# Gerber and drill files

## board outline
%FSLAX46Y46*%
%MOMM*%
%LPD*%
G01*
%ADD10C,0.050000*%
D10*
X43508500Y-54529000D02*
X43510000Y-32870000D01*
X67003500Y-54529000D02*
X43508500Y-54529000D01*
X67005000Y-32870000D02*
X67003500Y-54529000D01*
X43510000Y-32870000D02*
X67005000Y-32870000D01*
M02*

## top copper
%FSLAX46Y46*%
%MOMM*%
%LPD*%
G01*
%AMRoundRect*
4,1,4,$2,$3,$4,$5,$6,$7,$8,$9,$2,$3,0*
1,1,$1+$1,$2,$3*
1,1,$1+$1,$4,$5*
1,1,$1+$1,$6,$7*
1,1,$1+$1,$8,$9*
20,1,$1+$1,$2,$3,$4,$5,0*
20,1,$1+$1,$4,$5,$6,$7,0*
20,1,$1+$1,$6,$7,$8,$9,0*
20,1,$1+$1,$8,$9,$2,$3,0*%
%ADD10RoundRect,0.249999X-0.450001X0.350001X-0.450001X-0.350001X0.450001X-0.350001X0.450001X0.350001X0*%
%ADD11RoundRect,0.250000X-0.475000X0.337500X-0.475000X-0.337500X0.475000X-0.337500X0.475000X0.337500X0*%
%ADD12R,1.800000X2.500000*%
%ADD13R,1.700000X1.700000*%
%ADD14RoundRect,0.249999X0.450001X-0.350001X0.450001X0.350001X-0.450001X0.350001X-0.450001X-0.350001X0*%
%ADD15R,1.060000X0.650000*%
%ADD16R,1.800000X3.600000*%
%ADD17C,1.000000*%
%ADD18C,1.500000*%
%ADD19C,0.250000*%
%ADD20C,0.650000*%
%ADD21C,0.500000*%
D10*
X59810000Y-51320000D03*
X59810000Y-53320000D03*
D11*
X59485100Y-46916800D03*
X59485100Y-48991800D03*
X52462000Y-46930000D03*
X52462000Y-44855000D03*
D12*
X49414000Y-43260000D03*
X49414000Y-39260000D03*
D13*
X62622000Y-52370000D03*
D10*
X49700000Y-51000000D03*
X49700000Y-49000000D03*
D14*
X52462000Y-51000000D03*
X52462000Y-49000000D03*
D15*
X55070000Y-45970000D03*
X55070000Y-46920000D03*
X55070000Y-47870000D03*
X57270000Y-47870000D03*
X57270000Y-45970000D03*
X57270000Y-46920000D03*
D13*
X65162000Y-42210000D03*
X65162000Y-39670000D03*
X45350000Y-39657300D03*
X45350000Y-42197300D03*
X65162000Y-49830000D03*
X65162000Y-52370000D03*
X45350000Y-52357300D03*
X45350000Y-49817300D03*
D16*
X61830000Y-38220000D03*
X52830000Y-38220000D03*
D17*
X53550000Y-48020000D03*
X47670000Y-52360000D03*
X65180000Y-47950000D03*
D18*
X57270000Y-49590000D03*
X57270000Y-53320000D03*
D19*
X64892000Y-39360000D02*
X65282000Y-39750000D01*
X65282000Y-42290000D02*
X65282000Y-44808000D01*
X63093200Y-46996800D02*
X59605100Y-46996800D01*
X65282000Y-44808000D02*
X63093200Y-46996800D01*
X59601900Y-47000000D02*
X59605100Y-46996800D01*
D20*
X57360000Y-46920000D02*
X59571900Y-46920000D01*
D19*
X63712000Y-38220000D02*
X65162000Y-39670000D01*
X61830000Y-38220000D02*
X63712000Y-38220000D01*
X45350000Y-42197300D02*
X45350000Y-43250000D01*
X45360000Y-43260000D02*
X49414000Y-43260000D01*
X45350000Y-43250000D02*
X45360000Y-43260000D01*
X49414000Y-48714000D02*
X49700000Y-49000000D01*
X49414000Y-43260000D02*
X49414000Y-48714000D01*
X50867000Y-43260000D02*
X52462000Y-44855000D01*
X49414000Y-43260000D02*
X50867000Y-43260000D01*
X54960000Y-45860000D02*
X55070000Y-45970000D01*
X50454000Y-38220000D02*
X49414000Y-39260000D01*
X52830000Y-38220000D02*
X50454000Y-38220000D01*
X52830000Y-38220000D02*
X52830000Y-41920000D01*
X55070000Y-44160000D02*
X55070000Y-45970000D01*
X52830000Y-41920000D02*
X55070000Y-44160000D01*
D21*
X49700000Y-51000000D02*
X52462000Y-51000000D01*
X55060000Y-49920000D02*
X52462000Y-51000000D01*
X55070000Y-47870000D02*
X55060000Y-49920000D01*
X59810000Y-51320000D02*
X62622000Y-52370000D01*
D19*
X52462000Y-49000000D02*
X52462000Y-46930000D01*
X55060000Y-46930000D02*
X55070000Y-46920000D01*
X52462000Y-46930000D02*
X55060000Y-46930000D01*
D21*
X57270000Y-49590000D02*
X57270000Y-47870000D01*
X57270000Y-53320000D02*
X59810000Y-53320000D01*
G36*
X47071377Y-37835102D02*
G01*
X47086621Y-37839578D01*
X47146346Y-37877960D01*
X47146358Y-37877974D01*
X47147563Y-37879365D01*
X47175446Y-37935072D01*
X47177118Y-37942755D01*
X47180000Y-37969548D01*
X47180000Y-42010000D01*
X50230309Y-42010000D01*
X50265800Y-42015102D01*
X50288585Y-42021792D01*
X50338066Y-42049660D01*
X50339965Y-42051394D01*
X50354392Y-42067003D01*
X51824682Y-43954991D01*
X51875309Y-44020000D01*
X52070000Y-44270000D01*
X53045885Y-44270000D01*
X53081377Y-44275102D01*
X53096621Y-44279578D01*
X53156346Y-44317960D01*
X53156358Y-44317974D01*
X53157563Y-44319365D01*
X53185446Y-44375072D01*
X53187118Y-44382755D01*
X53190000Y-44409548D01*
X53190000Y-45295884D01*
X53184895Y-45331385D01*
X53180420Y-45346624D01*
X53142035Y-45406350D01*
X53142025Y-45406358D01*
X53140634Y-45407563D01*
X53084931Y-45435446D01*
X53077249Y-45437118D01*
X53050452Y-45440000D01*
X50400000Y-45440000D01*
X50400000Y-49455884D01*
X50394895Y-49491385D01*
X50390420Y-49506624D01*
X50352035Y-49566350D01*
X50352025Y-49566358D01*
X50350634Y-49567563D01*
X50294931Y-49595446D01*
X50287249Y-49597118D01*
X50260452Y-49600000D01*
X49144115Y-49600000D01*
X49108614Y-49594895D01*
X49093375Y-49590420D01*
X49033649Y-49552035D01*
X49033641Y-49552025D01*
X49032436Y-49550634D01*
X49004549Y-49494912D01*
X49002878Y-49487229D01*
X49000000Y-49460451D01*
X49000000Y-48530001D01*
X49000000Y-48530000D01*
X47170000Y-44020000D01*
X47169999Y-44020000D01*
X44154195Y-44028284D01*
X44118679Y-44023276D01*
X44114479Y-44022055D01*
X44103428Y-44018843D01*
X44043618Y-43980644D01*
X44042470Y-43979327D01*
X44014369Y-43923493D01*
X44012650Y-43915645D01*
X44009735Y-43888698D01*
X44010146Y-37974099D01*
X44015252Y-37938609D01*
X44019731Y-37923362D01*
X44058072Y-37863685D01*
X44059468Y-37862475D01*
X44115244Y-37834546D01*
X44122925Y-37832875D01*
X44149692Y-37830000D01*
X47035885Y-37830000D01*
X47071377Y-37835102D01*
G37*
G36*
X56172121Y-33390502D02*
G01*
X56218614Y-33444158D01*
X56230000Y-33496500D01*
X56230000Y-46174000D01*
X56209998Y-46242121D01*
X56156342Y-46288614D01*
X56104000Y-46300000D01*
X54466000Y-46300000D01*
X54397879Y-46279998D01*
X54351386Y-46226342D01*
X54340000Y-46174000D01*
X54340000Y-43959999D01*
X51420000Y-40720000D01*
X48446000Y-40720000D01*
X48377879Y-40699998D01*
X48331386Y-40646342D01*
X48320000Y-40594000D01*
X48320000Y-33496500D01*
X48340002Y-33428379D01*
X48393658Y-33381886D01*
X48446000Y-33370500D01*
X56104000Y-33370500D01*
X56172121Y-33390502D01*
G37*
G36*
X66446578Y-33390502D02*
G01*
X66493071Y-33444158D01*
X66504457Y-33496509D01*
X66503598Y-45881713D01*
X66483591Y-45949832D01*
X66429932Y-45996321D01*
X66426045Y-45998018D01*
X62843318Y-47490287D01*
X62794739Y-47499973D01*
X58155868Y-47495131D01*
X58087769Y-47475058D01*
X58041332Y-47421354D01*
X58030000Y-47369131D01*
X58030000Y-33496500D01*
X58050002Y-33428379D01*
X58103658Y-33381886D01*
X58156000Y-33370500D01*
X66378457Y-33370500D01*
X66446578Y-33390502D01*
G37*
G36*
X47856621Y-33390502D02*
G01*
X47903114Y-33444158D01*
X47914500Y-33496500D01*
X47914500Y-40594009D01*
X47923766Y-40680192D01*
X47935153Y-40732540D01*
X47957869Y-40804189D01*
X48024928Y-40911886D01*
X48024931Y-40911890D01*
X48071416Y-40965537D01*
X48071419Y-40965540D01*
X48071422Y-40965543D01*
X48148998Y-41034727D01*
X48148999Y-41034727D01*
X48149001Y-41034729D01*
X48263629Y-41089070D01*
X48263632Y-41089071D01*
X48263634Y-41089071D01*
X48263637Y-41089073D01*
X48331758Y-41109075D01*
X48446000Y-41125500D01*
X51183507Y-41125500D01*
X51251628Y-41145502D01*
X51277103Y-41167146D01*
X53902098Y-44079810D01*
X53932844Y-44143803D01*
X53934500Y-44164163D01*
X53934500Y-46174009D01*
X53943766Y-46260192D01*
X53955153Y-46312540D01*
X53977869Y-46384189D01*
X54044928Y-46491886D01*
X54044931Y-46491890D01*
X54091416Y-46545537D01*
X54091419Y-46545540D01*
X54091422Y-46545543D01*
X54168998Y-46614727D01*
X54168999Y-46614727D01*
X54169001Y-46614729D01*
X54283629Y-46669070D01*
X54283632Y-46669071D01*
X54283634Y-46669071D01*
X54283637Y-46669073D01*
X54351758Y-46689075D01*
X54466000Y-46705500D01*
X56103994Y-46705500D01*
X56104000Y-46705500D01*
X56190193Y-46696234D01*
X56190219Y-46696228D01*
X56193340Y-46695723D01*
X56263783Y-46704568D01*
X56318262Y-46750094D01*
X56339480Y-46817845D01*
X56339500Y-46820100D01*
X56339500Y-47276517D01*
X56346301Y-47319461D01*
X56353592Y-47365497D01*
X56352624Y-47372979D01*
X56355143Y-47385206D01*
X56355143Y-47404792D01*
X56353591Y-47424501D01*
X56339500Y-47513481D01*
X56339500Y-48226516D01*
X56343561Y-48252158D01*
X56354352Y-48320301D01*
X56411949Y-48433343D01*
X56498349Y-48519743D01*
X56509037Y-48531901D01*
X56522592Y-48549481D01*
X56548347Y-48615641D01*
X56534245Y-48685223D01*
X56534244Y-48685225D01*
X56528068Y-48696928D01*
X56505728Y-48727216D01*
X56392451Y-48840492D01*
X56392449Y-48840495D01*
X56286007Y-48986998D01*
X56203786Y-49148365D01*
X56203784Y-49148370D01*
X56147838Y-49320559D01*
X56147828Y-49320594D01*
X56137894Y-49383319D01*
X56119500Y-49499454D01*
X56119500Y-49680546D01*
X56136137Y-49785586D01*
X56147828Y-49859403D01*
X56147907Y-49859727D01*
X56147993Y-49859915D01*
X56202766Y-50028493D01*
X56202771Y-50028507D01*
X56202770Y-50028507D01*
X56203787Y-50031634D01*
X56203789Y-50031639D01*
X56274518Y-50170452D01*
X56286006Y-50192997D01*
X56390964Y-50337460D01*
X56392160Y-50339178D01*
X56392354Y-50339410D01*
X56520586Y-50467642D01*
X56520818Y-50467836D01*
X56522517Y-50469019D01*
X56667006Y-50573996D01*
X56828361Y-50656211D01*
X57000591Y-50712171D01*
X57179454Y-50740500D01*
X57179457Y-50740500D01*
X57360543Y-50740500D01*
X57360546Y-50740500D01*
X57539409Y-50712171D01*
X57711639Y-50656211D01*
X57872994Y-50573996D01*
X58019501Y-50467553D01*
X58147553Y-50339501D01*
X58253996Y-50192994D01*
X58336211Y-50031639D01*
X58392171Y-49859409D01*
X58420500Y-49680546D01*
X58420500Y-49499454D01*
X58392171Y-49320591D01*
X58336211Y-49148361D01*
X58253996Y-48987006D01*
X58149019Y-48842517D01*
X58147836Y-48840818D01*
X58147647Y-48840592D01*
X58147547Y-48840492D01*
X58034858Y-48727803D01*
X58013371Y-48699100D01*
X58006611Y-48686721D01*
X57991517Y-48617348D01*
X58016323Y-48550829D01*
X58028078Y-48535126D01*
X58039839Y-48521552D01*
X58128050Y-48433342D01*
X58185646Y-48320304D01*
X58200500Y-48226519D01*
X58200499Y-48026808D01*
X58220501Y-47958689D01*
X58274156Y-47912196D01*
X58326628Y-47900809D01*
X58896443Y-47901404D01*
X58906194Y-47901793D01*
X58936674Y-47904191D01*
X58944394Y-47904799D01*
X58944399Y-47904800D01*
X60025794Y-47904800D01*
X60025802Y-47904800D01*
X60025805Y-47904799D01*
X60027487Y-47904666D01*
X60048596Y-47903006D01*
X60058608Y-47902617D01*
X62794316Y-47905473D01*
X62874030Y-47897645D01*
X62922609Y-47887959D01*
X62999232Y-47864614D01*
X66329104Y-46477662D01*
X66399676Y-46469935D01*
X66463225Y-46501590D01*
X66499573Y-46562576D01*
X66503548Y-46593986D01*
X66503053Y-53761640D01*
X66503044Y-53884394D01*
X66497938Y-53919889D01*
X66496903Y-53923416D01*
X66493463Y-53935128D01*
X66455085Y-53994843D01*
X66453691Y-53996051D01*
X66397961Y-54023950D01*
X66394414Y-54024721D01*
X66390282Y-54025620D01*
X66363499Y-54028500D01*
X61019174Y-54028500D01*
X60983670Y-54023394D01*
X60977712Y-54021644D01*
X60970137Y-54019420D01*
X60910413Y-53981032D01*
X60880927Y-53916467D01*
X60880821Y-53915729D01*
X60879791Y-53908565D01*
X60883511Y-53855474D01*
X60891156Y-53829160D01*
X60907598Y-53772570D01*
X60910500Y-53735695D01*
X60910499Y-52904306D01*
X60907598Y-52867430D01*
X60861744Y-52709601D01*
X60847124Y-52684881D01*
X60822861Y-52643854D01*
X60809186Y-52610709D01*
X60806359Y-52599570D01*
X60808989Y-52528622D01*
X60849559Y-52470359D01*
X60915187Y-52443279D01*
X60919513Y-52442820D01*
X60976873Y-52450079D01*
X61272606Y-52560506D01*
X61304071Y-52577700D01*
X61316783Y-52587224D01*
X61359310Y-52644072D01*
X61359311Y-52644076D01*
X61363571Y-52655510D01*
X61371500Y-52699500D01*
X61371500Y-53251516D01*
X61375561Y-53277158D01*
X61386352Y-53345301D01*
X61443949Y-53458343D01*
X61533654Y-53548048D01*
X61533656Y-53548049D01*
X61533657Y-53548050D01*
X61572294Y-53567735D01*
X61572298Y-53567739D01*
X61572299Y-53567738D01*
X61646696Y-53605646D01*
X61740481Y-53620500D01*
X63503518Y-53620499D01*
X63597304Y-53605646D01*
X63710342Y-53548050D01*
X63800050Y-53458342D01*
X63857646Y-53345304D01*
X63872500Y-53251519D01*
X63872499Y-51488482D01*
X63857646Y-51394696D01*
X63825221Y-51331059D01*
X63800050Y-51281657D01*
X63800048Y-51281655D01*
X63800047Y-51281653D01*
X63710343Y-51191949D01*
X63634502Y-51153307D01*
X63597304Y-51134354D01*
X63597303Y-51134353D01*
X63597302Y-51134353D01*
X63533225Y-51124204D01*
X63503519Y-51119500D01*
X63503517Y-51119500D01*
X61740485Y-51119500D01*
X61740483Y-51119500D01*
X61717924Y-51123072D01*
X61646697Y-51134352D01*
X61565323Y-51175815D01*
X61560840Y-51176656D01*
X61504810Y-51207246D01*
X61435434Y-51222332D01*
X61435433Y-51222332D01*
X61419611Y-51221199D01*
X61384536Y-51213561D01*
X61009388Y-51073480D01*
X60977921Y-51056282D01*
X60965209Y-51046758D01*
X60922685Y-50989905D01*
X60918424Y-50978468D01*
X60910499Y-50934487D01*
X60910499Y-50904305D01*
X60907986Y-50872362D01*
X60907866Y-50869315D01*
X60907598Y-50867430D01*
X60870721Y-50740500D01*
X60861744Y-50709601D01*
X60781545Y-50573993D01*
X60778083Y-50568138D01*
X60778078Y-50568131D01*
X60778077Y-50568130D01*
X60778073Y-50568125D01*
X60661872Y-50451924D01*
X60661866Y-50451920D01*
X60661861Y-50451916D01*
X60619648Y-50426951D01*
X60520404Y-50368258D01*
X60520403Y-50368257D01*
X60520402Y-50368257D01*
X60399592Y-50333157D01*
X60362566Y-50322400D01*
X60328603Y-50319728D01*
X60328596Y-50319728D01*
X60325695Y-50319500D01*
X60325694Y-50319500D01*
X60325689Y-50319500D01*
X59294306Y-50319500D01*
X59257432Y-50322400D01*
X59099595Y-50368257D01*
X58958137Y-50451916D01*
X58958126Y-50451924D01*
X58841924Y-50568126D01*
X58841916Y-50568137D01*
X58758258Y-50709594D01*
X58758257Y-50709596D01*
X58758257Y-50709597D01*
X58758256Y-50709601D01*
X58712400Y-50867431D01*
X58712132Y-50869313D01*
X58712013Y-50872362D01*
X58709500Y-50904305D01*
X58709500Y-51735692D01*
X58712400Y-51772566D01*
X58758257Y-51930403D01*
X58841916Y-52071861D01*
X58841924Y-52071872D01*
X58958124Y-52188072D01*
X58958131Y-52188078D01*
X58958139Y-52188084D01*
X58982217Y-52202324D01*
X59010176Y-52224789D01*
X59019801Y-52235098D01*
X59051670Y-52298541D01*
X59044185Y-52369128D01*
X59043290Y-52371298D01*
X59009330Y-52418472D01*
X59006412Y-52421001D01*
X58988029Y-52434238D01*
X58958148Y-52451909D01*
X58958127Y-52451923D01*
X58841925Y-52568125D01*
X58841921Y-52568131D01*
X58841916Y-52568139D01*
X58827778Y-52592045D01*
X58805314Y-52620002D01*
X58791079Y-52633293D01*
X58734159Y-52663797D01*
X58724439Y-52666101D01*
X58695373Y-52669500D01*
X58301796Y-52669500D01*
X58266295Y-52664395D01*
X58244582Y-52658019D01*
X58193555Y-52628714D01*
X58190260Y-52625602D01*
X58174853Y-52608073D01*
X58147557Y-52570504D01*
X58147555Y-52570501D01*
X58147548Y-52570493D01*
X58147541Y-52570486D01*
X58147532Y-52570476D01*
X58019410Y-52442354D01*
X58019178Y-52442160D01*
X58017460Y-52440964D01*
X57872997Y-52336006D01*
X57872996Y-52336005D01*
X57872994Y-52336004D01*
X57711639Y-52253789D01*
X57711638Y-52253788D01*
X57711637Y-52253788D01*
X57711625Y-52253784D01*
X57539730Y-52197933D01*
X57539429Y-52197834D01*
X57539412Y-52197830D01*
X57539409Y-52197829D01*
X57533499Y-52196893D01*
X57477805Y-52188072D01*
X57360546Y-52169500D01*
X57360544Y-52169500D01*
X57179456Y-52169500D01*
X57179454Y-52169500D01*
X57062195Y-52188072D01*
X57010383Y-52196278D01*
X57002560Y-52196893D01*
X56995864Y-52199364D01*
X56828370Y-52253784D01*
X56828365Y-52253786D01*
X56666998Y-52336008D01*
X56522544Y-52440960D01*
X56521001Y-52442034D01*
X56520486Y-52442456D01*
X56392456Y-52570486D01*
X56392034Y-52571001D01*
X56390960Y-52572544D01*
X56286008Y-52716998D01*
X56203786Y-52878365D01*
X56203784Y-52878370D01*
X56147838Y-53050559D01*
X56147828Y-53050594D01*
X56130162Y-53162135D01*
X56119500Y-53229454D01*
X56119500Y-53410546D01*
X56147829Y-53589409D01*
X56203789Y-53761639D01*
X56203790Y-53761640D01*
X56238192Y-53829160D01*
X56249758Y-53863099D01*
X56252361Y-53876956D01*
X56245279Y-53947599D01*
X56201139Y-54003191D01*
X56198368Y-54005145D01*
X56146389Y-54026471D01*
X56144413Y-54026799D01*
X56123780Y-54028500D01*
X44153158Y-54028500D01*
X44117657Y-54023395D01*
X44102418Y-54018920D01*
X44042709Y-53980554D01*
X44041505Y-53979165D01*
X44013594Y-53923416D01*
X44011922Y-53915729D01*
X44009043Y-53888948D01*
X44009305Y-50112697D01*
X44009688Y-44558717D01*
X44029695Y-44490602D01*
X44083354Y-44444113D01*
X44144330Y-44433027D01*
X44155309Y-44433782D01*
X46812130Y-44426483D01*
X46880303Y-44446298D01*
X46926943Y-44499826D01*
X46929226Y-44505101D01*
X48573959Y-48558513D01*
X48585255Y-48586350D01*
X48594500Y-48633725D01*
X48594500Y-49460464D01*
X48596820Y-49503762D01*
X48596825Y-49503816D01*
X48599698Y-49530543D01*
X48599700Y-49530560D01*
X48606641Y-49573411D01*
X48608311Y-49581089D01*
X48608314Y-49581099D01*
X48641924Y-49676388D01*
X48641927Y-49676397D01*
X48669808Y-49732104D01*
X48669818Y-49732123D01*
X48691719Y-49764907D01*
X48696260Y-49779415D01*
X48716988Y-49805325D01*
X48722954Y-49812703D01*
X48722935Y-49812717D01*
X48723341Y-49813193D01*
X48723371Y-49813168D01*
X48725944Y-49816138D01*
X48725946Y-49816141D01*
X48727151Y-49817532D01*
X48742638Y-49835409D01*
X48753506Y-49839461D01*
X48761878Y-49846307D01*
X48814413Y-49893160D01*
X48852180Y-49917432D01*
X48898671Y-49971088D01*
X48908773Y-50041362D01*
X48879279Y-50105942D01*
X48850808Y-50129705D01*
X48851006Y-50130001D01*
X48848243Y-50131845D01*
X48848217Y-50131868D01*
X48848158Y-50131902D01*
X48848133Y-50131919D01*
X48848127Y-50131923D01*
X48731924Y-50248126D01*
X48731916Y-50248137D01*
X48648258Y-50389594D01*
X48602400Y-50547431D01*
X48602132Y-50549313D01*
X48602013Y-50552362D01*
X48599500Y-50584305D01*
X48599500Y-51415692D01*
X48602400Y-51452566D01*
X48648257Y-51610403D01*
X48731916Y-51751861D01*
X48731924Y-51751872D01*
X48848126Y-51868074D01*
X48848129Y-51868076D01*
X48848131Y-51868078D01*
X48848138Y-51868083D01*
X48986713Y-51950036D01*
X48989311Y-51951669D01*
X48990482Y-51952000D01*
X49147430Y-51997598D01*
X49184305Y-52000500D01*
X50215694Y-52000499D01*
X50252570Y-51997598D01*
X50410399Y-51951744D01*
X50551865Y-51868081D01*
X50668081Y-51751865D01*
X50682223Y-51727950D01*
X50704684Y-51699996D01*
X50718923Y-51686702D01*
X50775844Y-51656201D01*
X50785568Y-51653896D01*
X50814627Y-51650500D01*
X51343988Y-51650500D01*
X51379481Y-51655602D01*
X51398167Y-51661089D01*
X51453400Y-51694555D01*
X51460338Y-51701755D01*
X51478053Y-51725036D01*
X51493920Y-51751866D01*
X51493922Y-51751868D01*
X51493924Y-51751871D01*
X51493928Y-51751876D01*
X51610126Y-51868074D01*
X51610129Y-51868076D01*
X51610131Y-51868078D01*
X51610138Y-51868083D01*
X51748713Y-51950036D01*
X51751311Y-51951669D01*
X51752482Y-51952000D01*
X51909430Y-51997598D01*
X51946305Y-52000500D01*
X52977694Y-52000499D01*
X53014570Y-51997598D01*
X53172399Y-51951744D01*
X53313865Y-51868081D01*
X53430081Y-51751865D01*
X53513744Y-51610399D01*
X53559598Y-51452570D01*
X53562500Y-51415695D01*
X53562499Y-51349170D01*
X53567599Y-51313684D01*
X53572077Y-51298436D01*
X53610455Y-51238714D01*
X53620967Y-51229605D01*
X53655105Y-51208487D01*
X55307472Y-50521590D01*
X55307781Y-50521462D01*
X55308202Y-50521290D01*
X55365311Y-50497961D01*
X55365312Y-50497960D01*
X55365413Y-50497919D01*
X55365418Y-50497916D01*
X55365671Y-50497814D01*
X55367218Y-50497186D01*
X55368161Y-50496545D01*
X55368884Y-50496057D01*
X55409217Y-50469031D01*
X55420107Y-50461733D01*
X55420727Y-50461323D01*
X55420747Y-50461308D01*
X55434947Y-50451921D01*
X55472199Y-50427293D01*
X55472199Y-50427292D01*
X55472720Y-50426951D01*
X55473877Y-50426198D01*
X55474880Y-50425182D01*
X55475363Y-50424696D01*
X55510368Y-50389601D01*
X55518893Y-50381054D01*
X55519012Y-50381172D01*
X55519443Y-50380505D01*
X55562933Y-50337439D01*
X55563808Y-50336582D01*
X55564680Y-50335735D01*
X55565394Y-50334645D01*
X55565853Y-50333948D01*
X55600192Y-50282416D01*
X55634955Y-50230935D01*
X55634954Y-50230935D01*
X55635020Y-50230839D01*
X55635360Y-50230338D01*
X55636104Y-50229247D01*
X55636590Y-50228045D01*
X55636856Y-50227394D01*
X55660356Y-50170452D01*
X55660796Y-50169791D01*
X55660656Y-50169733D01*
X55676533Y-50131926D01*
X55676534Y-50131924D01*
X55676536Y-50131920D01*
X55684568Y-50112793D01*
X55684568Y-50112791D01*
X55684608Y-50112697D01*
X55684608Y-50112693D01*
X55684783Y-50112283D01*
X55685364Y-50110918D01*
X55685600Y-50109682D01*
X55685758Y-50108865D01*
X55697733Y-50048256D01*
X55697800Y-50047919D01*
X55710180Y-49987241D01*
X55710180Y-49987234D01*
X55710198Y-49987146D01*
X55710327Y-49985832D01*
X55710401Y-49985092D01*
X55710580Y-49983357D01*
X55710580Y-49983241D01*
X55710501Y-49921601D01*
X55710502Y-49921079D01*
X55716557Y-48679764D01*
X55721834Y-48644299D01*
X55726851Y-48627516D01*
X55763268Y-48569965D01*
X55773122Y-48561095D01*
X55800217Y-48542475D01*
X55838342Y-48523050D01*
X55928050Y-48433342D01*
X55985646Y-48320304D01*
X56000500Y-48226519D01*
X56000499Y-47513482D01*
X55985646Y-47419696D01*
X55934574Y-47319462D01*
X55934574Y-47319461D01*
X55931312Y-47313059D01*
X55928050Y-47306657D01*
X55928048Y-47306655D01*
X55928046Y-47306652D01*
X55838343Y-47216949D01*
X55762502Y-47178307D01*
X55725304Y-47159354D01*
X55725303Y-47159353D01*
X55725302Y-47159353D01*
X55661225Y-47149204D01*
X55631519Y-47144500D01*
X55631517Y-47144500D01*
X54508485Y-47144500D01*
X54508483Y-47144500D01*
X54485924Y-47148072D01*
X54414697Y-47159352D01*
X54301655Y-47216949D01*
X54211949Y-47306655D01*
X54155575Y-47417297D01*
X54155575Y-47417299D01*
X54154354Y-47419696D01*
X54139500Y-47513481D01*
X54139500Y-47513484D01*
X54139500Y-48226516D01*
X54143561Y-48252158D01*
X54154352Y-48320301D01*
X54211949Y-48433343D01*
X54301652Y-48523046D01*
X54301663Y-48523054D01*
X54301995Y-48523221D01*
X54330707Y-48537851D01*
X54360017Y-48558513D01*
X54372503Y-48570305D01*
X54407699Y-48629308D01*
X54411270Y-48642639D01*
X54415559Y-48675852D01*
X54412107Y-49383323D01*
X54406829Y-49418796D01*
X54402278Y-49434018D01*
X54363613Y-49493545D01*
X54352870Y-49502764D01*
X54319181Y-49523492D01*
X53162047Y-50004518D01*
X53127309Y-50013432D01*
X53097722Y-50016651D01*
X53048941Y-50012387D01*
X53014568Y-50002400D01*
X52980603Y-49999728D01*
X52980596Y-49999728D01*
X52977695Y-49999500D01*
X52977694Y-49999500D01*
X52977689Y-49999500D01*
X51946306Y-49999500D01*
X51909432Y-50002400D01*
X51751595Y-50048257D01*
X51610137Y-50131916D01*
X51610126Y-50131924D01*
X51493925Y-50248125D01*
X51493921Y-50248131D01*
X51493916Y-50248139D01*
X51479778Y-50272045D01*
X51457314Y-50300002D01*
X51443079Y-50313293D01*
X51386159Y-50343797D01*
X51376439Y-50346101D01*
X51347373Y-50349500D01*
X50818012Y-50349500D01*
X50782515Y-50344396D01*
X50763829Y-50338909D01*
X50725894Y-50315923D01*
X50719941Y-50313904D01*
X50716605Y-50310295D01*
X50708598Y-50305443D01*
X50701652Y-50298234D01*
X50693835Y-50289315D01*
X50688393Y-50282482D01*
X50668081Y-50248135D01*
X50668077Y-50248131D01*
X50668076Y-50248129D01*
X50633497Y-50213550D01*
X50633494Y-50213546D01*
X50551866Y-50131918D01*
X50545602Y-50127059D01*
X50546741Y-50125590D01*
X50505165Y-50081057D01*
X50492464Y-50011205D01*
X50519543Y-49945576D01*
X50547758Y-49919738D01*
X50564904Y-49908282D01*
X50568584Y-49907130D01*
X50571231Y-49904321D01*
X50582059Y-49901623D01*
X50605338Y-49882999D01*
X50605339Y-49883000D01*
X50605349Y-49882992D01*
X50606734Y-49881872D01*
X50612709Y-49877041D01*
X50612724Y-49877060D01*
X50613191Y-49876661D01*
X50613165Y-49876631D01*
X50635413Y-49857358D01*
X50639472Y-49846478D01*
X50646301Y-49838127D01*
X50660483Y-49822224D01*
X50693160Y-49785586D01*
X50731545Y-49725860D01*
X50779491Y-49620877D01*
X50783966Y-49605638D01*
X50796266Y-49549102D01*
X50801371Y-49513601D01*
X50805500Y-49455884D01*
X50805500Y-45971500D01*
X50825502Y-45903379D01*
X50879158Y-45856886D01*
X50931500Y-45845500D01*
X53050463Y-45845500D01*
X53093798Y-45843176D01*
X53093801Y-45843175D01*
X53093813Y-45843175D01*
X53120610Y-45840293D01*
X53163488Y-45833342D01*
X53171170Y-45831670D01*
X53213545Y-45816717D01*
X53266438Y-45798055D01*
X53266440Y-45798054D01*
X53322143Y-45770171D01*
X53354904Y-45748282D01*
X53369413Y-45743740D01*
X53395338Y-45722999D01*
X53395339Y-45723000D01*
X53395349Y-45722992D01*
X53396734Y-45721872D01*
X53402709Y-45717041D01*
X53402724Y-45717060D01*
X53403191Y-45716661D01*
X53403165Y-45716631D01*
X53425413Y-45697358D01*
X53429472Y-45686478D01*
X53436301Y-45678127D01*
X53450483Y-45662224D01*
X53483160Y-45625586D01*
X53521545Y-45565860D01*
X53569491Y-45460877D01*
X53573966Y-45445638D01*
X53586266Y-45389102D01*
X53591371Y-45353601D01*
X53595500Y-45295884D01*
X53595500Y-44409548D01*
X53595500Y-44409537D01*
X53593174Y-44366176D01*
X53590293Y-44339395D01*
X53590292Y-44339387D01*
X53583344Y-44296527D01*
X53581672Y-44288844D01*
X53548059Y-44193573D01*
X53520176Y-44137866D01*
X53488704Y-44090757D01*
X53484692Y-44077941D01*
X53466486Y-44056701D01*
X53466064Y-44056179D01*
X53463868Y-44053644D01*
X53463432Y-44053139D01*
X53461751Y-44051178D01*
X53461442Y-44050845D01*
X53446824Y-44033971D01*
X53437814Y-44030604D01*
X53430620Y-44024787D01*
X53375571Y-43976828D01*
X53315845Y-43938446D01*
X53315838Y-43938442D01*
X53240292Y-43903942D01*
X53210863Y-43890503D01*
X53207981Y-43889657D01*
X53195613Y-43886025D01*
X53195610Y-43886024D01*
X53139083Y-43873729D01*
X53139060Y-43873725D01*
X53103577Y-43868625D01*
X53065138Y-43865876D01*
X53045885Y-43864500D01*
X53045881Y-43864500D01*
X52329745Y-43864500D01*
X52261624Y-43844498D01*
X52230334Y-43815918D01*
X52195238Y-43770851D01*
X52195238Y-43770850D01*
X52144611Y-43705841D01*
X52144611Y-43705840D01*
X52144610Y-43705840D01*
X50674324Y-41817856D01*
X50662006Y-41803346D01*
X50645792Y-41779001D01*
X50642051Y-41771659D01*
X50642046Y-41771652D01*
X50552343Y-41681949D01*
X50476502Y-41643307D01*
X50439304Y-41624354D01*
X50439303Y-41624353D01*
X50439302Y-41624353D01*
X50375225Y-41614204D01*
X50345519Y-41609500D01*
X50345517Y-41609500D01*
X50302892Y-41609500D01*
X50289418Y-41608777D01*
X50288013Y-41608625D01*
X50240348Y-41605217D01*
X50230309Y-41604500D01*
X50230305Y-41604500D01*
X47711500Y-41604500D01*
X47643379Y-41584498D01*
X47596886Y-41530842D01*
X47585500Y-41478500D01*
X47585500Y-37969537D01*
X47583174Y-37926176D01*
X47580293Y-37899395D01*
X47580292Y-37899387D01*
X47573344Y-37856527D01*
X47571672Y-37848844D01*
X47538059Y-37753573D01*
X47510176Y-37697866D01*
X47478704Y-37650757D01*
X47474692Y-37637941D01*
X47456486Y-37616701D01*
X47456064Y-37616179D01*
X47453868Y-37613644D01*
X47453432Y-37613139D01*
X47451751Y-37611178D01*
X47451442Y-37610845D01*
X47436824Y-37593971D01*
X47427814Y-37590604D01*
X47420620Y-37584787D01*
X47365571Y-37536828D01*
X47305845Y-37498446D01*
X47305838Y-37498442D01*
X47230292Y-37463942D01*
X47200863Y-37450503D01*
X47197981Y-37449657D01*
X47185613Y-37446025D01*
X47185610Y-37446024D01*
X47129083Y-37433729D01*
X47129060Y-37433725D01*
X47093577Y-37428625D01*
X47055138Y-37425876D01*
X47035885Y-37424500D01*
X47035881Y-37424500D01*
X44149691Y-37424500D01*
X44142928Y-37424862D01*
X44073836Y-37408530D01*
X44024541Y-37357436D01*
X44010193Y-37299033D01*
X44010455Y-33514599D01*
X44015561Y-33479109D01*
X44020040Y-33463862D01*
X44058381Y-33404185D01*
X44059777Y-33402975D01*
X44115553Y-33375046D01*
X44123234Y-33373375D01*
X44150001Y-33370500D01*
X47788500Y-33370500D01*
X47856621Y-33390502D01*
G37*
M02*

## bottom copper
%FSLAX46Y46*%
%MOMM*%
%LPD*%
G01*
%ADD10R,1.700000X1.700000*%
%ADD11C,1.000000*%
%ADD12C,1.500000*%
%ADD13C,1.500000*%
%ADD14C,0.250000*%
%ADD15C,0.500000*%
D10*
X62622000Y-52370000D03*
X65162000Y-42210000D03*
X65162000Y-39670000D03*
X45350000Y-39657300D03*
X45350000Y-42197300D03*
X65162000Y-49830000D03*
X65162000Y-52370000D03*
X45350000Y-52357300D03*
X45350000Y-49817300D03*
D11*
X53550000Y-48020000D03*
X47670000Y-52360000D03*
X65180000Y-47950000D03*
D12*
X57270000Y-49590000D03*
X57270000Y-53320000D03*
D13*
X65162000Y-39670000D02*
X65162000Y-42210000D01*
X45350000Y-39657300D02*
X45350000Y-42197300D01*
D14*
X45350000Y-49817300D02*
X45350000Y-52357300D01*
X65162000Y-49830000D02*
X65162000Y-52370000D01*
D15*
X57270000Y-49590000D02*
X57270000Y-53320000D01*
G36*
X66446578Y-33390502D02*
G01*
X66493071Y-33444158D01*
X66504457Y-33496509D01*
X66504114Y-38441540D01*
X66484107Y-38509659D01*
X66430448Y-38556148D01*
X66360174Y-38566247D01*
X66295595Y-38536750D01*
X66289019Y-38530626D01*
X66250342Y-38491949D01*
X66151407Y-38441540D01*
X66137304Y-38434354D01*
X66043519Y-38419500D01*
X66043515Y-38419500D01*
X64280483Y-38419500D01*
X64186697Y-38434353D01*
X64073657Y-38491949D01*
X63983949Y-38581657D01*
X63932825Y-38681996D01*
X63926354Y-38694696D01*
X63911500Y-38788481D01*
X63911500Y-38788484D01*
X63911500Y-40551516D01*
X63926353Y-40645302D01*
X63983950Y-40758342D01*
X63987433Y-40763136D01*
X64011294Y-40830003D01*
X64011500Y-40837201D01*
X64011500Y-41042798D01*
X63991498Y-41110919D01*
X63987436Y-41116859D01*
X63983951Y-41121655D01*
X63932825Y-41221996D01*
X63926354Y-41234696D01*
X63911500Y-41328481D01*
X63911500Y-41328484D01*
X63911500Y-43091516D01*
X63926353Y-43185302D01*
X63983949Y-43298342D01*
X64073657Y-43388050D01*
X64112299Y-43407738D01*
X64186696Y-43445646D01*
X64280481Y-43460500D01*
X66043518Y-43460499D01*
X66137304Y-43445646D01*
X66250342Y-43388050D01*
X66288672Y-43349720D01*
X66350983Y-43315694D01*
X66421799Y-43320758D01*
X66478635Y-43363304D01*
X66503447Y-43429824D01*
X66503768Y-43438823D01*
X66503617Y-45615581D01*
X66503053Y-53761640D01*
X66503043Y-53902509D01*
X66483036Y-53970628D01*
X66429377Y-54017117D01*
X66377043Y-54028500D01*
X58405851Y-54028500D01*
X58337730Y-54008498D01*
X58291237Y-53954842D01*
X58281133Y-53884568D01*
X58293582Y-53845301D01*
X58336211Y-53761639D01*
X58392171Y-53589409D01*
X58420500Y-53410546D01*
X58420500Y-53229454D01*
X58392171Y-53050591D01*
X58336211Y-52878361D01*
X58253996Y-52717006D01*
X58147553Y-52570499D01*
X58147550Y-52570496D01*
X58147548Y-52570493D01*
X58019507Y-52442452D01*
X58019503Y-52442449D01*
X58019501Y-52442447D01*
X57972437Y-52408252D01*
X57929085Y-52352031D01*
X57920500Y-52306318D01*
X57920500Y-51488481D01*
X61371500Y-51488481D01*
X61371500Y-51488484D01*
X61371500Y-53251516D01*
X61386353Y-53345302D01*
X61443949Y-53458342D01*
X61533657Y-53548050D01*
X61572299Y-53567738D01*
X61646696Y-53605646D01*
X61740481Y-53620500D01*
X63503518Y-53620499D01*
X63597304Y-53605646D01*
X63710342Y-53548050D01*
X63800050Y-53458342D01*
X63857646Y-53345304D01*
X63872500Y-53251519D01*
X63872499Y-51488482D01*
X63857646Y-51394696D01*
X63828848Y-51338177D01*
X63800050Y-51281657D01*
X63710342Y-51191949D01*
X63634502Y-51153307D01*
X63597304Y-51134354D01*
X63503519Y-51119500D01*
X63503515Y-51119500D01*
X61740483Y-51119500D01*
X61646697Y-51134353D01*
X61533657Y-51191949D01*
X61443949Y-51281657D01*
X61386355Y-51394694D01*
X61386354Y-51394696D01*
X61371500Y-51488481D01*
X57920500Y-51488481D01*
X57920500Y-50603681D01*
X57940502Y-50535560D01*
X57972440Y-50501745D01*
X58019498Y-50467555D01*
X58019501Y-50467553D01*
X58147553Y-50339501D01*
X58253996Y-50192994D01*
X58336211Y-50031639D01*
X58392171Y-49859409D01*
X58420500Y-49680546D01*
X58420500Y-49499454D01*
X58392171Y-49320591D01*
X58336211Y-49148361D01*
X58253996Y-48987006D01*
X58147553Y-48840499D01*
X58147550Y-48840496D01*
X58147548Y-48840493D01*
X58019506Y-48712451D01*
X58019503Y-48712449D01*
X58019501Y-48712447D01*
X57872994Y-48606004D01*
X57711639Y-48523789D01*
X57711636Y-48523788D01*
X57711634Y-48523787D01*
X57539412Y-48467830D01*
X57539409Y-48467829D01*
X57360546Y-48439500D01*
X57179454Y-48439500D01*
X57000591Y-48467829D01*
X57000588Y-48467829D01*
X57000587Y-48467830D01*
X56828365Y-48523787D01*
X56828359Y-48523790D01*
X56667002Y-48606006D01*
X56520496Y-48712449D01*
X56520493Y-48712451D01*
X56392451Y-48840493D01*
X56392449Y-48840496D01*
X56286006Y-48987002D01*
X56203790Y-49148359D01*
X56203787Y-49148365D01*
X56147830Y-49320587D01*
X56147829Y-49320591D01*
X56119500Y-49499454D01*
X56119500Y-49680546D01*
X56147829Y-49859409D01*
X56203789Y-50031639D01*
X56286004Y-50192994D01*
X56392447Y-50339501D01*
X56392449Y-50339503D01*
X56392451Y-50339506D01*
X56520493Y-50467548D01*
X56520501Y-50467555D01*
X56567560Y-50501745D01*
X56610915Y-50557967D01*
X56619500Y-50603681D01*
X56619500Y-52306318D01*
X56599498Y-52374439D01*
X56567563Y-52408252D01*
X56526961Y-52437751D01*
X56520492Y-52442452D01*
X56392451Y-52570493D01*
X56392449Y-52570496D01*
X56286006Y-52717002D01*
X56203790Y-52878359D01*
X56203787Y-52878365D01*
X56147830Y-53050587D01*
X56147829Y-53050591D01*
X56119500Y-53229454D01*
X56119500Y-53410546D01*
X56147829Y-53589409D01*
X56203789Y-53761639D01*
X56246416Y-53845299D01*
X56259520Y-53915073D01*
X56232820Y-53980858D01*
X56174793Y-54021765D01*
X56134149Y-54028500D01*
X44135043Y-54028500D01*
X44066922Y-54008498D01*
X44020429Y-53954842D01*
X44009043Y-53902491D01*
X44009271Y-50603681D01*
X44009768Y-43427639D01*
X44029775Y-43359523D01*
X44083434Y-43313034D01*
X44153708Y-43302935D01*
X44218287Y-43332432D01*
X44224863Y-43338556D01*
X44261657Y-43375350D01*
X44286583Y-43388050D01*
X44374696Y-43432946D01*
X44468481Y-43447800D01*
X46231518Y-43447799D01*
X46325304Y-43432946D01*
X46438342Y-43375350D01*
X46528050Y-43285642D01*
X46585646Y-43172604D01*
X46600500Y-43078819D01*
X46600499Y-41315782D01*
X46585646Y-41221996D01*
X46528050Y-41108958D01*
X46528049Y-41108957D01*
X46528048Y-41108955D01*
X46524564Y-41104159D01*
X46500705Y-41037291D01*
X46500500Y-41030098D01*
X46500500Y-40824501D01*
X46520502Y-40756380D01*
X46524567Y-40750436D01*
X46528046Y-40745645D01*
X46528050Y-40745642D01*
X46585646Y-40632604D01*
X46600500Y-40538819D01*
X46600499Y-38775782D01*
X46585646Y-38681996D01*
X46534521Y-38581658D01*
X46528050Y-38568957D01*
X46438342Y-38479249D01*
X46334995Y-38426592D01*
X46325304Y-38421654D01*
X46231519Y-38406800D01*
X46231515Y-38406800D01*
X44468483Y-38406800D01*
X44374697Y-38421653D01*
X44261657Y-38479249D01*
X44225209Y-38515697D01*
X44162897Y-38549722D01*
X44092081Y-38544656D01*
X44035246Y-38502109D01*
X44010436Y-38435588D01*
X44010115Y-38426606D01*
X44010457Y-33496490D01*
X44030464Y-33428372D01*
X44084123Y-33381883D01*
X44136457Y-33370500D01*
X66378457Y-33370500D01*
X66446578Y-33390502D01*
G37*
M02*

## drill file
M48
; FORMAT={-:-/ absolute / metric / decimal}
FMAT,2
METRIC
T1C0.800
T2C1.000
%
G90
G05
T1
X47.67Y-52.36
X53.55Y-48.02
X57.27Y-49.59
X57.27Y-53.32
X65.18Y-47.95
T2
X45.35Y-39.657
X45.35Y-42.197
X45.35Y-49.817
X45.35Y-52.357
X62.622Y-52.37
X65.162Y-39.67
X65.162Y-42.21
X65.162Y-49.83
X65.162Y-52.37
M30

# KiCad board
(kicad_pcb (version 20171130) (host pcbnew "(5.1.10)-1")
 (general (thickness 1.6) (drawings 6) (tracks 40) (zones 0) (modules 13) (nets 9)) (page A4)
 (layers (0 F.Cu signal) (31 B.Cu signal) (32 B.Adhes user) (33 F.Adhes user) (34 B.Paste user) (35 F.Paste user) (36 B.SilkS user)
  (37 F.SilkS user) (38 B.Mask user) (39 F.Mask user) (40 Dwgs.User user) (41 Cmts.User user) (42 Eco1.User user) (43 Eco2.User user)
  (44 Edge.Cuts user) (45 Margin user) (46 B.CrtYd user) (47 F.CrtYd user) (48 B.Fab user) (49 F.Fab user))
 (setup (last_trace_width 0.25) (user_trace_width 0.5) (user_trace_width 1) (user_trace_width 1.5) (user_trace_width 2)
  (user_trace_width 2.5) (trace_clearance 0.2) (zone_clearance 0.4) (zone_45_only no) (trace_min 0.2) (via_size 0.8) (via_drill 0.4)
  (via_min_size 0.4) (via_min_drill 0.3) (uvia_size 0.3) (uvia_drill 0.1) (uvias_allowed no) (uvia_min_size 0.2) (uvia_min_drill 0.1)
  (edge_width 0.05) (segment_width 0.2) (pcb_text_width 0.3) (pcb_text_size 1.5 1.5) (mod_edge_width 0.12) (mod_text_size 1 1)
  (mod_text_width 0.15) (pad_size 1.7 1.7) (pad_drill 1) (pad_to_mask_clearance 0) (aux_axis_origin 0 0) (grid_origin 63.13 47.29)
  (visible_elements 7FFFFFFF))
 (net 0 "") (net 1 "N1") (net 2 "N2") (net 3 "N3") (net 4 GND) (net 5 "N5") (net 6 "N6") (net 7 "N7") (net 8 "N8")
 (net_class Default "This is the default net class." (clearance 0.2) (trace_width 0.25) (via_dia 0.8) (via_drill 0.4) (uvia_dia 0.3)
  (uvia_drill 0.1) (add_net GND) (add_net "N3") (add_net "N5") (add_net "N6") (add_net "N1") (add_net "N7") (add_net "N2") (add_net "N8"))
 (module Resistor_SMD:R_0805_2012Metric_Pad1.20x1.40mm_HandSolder (layer F.Cu) (at 59.81 52.32 270)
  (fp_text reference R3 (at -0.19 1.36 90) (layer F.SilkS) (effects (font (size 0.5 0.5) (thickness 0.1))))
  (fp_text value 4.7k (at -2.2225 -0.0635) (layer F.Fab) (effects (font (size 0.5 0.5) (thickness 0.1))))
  (pad 1 smd roundrect (at -1 0 270) (size 1.2 1.4) (layers F.Cu F.Paste F.Mask) (roundrect_rratio 0.2083325) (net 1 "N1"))
  (pad 2 smd roundrect (at 1 0 270) (size 1.2 1.4) (layers F.Cu F.Paste F.Mask) (roundrect_rratio 0.2083325) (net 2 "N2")))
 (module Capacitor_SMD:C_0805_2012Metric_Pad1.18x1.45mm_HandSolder (layer F.Cu) (at 59.4851 47.9543 270)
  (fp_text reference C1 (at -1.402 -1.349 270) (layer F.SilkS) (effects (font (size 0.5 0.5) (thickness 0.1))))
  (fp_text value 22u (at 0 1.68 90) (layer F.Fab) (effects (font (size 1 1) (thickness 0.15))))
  (pad 1 smd roundrect (at -1.0375 0 270) (size 1.175 1.45) (layers F.Cu F.Paste F.Mask) (roundrect_rratio 0.2127659574468085) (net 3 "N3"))
  (pad 2 smd roundrect (at 1.0375 0 270) (size 1.175 1.45) (layers F.Cu F.Paste F.Mask) (roundrect_rratio 0.2127659574468085) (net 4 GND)))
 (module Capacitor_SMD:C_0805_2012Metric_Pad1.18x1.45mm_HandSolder (layer F.Cu) (at 52.462 45.8925 270)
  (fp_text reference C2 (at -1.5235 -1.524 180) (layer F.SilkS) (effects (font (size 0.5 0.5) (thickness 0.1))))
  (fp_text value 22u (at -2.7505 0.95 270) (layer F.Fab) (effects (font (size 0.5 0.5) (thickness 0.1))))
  (pad 2 smd roundrect (at 1.0375 0 270) (size 1.175 1.45) (layers F.Cu F.Paste F.Mask) (roundrect_rratio 0.2127659574468085) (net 4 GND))
  (pad 1 smd roundrect (at -1.0375 0 270) (size 1.175 1.45) (layers F.Cu F.Paste F.Mask) (roundrect_rratio 0.2127659574468085) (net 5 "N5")))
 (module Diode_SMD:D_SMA (layer F.Cu) (at 49.414 41.26 90)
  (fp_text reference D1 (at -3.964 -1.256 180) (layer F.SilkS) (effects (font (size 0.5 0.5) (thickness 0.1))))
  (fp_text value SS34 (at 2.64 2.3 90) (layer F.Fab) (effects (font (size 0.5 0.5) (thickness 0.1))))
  (pad 1 smd rect (at -2 0 90) (size 2.5 1.8) (layers F.Cu F.Paste F.Mask) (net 5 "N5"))
  (pad 2 smd rect (at 2 0 90) (size 2.5 1.8) (layers F.Cu F.Paste F.Mask) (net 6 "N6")))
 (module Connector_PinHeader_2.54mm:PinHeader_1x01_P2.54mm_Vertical (layer F.Cu) (at 62.622 52.37 180)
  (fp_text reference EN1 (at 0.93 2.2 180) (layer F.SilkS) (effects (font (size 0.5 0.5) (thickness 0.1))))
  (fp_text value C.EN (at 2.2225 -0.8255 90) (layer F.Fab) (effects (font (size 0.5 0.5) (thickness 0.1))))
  (pad 1 thru_hole rect (at 0 0 180) (size 1.7 1.7) (drill 1) (layers *.Cu *.Mask) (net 1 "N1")))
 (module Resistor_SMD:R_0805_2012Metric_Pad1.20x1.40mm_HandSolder (layer F.Cu) (at 49.7 50 270)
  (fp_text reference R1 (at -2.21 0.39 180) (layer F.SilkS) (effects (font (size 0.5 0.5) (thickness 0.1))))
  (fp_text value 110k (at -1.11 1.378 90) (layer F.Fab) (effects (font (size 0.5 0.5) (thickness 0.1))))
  (pad 2 smd roundrect (at 1 0 270) (size 1.2 1.4) (layers F.Cu F.Paste F.Mask) (roundrect_rratio 0.2083325) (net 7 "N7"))
  (pad 1 smd roundrect (at -1 0 270) (size 1.2 1.4) (layers F.Cu F.Paste F.Mask) (roundrect_rratio 0.2083325) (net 5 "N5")))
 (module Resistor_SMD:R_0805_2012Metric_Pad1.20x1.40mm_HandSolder (layer F.Cu) (at 52.462 50 90)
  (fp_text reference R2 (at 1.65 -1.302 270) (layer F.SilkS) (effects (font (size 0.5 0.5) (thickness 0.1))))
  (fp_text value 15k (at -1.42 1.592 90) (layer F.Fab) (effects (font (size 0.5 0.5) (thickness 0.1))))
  (pad 1 smd roundrect (at -1 0 90) (size 1.2 1.4) (layers F.Cu F.Paste F.Mask) (roundrect_rratio 0.2083325) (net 7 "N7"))
  (pad 2 smd roundrect (at 1 0 90) (size 1.2 1.4) (layers F.Cu F.Paste F.Mask) (roundrect_rratio 0.2083325) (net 4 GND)))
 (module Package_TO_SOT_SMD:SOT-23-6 (layer F.Cu) (at 56.17 46.92) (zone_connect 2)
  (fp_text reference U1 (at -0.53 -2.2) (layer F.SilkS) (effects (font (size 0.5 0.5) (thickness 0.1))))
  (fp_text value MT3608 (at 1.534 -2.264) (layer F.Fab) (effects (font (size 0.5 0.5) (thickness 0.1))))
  (pad 1 smd rect (at -1.1 -0.95) (size 1.06 0.65) (layers F.Cu F.Paste F.Mask) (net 6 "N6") (zone_connect 2))
  (pad 2 smd rect (at -1.1 0) (size 1.06 0.65) (layers F.Cu F.Paste F.Mask) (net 4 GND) (zone_connect 2))
  (pad 3 smd rect (at -1.1 0.95) (size 1.06 0.65) (layers F.Cu F.Paste F.Mask) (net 7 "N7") (zone_connect 2))
  (pad 4 smd rect (at 1.1 0.95) (size 1.06 0.65) (layers F.Cu F.Paste F.Mask) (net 2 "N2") (zone_connect 2))
  (pad 6 smd rect (at 1.1 -0.95) (size 1.06 0.65) (layers F.Cu F.Paste F.Mask) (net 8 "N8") (zone_connect 2))
  (pad 5 smd rect (at 1.1 0) (size 1.06 0.65) (layers F.Cu F.Paste F.Mask) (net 3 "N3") (zone_connect 2)))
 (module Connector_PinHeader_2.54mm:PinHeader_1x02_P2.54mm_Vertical (layer F.Cu) (at 65.162 39.67)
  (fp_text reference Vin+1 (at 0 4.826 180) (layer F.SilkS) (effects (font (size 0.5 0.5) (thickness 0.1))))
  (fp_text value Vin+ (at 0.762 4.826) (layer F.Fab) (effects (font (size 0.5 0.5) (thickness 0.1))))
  (pad 2 thru_hole rect (at 0 2.54) (size 1.7 1.7) (drill 1) (layers *.Cu *.Mask) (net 3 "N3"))
  (pad 1 thru_hole rect (at 0 0) (size 1.7 1.7) (drill 1) (layers *.Cu *.Mask) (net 3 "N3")))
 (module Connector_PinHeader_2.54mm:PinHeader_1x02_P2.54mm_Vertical (layer F.Cu) (at 45.35 39.6573)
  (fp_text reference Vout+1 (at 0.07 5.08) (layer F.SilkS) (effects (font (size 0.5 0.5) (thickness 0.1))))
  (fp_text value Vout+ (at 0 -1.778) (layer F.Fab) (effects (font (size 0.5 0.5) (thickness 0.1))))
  (pad 1 thru_hole rect (at 0 0) (size 1.7 1.7) (drill 1) (layers *.Cu *.Mask) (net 5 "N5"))
  (pad 2 thru_hole rect (at 0 2.54) (size 1.7 1.7) (drill 1) (layers *.Cu *.Mask) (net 5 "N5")))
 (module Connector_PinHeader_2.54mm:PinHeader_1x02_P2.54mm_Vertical (layer F.Cu) (at 65.162 49.83)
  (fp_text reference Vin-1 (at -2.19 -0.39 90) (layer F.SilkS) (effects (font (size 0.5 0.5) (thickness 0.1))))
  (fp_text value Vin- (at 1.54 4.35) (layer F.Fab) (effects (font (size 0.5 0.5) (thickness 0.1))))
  (pad 1 thru_hole rect (at 0 0) (size 1.7 1.7) (drill 1) (layers *.Cu *.Mask) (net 4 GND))
  (pad 2 thru_hole rect (at 0 2.54) (size 1.7 1.7) (drill 1) (layers *.Cu *.Mask) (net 4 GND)))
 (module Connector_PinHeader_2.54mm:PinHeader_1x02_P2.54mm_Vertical (layer F.Cu) (at 45.35 49.8173)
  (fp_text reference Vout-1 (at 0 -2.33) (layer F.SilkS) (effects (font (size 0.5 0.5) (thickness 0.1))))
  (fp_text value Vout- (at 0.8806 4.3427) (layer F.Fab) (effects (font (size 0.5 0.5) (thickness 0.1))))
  (pad 2 thru_hole rect (at 0 2.54) (size 1.7 1.7) (drill 1) (layers *.Cu *.Mask) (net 4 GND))
  (pad 1 thru_hole rect (at 0 0) (size 1.7 1.7) (drill 1) (layers *.Cu *.Mask) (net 4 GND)))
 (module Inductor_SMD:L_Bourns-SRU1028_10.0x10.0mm (layer F.Cu) (at 57.33 38.22 180)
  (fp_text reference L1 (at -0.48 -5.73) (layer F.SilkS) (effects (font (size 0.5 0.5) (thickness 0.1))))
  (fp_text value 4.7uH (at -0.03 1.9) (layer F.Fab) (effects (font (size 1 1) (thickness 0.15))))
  (pad 1 smd rect (at -4.5 0 180) (size 1.8 3.6) (layers F.Cu F.Paste F.Mask) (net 3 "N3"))
  (pad 2 smd rect (at 4.5 0 180) (size 1.8 3.6) (layers F.Cu F.Paste F.Mask) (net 6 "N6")))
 (gr_line (start 43.5085 54.529) (end 43.51 32.87) (layer Edge.Cuts) (width 0.05))
 (gr_line (start 67.0035 54.529) (end 43.5085 54.529) (layer Edge.Cuts) (width 0.05))
 (gr_line (start 67.005 32.87) (end 67.0035 54.529) (layer Edge.Cuts) (width 0.05))
 (gr_line (start 43.51 32.87) (end 67.005 32.87) (layer Edge.Cuts) (width 0.05))
 (segment (start 64.892 39.36) (end 65.282 39.75) (width 0.25) (layer F.Cu) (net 3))
 (segment (start 65.282 42.29) (end 65.282 44.808) (width 0.25) (layer F.Cu) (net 3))
 (segment (start 63.0932 46.9968) (end 59.6051 46.9968) (width 0.25) (layer F.Cu) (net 3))
 (segment (start 65.282 44.808) (end 63.0932 46.9968) (width 0.25) (layer F.Cu) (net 3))
 (segment (start 59.6019 47) (end 59.6051 46.9968) (width 0.25) (layer F.Cu) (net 3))
 (segment (start 57.36 46.92) (end 59.5719 46.92) (width 0.65) (layer F.Cu) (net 3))
 (segment (start 65.162 39.67) (end 65.162 42.21) (width 1.5) (layer B.Cu) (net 3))
 (segment (start 63.712 38.22) (end 65.162 39.67) (width 0.25) (layer F.Cu) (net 3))
 (segment (start 61.83 38.22) (end 63.712 38.22) (width 0.25) (layer F.Cu) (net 3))
 (segment (start 45.35 42.1973) (end 45.35 43.25) (width 0.25) (layer F.Cu) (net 5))
 (segment (start 45.36 43.26) (end 49.414 43.26) (width 0.25) (layer F.Cu) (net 5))
 (segment (start 45.35 43.25) (end 45.36 43.26) (width 0.25) (layer F.Cu) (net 5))
 (segment (start 49.414 48.714) (end 49.7 49) (width 0.25) (layer F.Cu) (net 5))
 (segment (start 49.414 43.26) (end 49.414 48.714) (width 0.25) (layer F.Cu) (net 5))
 (segment (start 50.867 43.26) (end 52.462 44.855) (width 0.25) (layer F.Cu) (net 5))
 (segment (start 49.414 43.26) (end 50.867 43.26) (width 0.25) (layer F.Cu) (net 5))
 (segment (start 45.35 39.6573) (end 45.35 42.1973) (width 1.5) (layer B.Cu) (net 5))
 (segment (start 54.96 45.86) (end 55.07 45.97) (width 0.25) (layer F.Cu) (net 6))
 (segment (start 50.454 38.22) (end 49.414 39.26) (width 0.25) (layer F.Cu) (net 6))
 (segment (start 52.83 38.22) (end 50.454 38.22) (width 0.25) (layer F.Cu) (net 6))
 (segment (start 52.83 38.22) (end 52.83 41.92) (width 0.25) (layer F.Cu) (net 6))
 (segment (start 55.07 44.16) (end 55.07 45.97) (width 0.25) (layer F.Cu) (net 6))
 (segment (start 52.83 41.92) (end 55.07 44.16) (width 0.25) (layer F.Cu) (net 6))
 (segment (start 49.7 51) (end 52.462 51) (width 0.5) (layer F.Cu) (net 7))
 (segment (start 55.06 49.92) (end 52.462 51) (width 0.5) (layer F.Cu) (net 7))
 (segment (start 55.07 47.87) (end 55.06 49.92) (width 0.5) (layer F.Cu) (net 7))
 (segment (start 59.81 51.32) (end 62.622 52.37) (width 0.5) (layer F.Cu) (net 1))
 (via (at 53.55 48.02) (size 1) (drill 0.8) (layers F.Cu B.Cu) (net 4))
 (via (at 47.67 52.36) (size 1) (drill 0.8) (layers F.Cu B.Cu) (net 4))
 (via (at 65.18 47.95) (size 1) (drill 0.8) (layers F.Cu B.Cu) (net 4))
 (segment (start 52.462 49) (end 52.462 46.93) (width 0.25) (layer F.Cu) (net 4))
 (segment (start 55.06 46.93) (end 55.07 46.92) (width 0.25) (layer F.Cu) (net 4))
 (segment (start 52.462 46.93) (end 55.06 46.93) (width 0.25) (layer F.Cu) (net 4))
 (segment (start 45.35 49.8173) (end 45.35 52.3573) (width 0.25) (layer B.Cu) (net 4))
 (segment (start 65.162 49.83) (end 65.162 52.37) (width 0.25) (layer B.Cu) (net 4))
 (via (at 57.27 49.59) (size 1.5) (drill 0.8) (layers F.Cu B.Cu) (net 2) (status 40000))
 (via (at 57.27 53.32) (size 1.5) (drill 0.8) (layers F.Cu B.Cu) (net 2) (status 40000))
 (segment (start 57.27 49.59) (end 57.27 47.87) (width 0.5) (layer F.Cu) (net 2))
 (segment (start 57.27 49.59) (end 57.27 53.32) (width 0.5) (layer B.Cu) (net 2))
 (segment (start 57.27 53.32) (end 59.81 53.32) (width 0.5) (layer F.Cu) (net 2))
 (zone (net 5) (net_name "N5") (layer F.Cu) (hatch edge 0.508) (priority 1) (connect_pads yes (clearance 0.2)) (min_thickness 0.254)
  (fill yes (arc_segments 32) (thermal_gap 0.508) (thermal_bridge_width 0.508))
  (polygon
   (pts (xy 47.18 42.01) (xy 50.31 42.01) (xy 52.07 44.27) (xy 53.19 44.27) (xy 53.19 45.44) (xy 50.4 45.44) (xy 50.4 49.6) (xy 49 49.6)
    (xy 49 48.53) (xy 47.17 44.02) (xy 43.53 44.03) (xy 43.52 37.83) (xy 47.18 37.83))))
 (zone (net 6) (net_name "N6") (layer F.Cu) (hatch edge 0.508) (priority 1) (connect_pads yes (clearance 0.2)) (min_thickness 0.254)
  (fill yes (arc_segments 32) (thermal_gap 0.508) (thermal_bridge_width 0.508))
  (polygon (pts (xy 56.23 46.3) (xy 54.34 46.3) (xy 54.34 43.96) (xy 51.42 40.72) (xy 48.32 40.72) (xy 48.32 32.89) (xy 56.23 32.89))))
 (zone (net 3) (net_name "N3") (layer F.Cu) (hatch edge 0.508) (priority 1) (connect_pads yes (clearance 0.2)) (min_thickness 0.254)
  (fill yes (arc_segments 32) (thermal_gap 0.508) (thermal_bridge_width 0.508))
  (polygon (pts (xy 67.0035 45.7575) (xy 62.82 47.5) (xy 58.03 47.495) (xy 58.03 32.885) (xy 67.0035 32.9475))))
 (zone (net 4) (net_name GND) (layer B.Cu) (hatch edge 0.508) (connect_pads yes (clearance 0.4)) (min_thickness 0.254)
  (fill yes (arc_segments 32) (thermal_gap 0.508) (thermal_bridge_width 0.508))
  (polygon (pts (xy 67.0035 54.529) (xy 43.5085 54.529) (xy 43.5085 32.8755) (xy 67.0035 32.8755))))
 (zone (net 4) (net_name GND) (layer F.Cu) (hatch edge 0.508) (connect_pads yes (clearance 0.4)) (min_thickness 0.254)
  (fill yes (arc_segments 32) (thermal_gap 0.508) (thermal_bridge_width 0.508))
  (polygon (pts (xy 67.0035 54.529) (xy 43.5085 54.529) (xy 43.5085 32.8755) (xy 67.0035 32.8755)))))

